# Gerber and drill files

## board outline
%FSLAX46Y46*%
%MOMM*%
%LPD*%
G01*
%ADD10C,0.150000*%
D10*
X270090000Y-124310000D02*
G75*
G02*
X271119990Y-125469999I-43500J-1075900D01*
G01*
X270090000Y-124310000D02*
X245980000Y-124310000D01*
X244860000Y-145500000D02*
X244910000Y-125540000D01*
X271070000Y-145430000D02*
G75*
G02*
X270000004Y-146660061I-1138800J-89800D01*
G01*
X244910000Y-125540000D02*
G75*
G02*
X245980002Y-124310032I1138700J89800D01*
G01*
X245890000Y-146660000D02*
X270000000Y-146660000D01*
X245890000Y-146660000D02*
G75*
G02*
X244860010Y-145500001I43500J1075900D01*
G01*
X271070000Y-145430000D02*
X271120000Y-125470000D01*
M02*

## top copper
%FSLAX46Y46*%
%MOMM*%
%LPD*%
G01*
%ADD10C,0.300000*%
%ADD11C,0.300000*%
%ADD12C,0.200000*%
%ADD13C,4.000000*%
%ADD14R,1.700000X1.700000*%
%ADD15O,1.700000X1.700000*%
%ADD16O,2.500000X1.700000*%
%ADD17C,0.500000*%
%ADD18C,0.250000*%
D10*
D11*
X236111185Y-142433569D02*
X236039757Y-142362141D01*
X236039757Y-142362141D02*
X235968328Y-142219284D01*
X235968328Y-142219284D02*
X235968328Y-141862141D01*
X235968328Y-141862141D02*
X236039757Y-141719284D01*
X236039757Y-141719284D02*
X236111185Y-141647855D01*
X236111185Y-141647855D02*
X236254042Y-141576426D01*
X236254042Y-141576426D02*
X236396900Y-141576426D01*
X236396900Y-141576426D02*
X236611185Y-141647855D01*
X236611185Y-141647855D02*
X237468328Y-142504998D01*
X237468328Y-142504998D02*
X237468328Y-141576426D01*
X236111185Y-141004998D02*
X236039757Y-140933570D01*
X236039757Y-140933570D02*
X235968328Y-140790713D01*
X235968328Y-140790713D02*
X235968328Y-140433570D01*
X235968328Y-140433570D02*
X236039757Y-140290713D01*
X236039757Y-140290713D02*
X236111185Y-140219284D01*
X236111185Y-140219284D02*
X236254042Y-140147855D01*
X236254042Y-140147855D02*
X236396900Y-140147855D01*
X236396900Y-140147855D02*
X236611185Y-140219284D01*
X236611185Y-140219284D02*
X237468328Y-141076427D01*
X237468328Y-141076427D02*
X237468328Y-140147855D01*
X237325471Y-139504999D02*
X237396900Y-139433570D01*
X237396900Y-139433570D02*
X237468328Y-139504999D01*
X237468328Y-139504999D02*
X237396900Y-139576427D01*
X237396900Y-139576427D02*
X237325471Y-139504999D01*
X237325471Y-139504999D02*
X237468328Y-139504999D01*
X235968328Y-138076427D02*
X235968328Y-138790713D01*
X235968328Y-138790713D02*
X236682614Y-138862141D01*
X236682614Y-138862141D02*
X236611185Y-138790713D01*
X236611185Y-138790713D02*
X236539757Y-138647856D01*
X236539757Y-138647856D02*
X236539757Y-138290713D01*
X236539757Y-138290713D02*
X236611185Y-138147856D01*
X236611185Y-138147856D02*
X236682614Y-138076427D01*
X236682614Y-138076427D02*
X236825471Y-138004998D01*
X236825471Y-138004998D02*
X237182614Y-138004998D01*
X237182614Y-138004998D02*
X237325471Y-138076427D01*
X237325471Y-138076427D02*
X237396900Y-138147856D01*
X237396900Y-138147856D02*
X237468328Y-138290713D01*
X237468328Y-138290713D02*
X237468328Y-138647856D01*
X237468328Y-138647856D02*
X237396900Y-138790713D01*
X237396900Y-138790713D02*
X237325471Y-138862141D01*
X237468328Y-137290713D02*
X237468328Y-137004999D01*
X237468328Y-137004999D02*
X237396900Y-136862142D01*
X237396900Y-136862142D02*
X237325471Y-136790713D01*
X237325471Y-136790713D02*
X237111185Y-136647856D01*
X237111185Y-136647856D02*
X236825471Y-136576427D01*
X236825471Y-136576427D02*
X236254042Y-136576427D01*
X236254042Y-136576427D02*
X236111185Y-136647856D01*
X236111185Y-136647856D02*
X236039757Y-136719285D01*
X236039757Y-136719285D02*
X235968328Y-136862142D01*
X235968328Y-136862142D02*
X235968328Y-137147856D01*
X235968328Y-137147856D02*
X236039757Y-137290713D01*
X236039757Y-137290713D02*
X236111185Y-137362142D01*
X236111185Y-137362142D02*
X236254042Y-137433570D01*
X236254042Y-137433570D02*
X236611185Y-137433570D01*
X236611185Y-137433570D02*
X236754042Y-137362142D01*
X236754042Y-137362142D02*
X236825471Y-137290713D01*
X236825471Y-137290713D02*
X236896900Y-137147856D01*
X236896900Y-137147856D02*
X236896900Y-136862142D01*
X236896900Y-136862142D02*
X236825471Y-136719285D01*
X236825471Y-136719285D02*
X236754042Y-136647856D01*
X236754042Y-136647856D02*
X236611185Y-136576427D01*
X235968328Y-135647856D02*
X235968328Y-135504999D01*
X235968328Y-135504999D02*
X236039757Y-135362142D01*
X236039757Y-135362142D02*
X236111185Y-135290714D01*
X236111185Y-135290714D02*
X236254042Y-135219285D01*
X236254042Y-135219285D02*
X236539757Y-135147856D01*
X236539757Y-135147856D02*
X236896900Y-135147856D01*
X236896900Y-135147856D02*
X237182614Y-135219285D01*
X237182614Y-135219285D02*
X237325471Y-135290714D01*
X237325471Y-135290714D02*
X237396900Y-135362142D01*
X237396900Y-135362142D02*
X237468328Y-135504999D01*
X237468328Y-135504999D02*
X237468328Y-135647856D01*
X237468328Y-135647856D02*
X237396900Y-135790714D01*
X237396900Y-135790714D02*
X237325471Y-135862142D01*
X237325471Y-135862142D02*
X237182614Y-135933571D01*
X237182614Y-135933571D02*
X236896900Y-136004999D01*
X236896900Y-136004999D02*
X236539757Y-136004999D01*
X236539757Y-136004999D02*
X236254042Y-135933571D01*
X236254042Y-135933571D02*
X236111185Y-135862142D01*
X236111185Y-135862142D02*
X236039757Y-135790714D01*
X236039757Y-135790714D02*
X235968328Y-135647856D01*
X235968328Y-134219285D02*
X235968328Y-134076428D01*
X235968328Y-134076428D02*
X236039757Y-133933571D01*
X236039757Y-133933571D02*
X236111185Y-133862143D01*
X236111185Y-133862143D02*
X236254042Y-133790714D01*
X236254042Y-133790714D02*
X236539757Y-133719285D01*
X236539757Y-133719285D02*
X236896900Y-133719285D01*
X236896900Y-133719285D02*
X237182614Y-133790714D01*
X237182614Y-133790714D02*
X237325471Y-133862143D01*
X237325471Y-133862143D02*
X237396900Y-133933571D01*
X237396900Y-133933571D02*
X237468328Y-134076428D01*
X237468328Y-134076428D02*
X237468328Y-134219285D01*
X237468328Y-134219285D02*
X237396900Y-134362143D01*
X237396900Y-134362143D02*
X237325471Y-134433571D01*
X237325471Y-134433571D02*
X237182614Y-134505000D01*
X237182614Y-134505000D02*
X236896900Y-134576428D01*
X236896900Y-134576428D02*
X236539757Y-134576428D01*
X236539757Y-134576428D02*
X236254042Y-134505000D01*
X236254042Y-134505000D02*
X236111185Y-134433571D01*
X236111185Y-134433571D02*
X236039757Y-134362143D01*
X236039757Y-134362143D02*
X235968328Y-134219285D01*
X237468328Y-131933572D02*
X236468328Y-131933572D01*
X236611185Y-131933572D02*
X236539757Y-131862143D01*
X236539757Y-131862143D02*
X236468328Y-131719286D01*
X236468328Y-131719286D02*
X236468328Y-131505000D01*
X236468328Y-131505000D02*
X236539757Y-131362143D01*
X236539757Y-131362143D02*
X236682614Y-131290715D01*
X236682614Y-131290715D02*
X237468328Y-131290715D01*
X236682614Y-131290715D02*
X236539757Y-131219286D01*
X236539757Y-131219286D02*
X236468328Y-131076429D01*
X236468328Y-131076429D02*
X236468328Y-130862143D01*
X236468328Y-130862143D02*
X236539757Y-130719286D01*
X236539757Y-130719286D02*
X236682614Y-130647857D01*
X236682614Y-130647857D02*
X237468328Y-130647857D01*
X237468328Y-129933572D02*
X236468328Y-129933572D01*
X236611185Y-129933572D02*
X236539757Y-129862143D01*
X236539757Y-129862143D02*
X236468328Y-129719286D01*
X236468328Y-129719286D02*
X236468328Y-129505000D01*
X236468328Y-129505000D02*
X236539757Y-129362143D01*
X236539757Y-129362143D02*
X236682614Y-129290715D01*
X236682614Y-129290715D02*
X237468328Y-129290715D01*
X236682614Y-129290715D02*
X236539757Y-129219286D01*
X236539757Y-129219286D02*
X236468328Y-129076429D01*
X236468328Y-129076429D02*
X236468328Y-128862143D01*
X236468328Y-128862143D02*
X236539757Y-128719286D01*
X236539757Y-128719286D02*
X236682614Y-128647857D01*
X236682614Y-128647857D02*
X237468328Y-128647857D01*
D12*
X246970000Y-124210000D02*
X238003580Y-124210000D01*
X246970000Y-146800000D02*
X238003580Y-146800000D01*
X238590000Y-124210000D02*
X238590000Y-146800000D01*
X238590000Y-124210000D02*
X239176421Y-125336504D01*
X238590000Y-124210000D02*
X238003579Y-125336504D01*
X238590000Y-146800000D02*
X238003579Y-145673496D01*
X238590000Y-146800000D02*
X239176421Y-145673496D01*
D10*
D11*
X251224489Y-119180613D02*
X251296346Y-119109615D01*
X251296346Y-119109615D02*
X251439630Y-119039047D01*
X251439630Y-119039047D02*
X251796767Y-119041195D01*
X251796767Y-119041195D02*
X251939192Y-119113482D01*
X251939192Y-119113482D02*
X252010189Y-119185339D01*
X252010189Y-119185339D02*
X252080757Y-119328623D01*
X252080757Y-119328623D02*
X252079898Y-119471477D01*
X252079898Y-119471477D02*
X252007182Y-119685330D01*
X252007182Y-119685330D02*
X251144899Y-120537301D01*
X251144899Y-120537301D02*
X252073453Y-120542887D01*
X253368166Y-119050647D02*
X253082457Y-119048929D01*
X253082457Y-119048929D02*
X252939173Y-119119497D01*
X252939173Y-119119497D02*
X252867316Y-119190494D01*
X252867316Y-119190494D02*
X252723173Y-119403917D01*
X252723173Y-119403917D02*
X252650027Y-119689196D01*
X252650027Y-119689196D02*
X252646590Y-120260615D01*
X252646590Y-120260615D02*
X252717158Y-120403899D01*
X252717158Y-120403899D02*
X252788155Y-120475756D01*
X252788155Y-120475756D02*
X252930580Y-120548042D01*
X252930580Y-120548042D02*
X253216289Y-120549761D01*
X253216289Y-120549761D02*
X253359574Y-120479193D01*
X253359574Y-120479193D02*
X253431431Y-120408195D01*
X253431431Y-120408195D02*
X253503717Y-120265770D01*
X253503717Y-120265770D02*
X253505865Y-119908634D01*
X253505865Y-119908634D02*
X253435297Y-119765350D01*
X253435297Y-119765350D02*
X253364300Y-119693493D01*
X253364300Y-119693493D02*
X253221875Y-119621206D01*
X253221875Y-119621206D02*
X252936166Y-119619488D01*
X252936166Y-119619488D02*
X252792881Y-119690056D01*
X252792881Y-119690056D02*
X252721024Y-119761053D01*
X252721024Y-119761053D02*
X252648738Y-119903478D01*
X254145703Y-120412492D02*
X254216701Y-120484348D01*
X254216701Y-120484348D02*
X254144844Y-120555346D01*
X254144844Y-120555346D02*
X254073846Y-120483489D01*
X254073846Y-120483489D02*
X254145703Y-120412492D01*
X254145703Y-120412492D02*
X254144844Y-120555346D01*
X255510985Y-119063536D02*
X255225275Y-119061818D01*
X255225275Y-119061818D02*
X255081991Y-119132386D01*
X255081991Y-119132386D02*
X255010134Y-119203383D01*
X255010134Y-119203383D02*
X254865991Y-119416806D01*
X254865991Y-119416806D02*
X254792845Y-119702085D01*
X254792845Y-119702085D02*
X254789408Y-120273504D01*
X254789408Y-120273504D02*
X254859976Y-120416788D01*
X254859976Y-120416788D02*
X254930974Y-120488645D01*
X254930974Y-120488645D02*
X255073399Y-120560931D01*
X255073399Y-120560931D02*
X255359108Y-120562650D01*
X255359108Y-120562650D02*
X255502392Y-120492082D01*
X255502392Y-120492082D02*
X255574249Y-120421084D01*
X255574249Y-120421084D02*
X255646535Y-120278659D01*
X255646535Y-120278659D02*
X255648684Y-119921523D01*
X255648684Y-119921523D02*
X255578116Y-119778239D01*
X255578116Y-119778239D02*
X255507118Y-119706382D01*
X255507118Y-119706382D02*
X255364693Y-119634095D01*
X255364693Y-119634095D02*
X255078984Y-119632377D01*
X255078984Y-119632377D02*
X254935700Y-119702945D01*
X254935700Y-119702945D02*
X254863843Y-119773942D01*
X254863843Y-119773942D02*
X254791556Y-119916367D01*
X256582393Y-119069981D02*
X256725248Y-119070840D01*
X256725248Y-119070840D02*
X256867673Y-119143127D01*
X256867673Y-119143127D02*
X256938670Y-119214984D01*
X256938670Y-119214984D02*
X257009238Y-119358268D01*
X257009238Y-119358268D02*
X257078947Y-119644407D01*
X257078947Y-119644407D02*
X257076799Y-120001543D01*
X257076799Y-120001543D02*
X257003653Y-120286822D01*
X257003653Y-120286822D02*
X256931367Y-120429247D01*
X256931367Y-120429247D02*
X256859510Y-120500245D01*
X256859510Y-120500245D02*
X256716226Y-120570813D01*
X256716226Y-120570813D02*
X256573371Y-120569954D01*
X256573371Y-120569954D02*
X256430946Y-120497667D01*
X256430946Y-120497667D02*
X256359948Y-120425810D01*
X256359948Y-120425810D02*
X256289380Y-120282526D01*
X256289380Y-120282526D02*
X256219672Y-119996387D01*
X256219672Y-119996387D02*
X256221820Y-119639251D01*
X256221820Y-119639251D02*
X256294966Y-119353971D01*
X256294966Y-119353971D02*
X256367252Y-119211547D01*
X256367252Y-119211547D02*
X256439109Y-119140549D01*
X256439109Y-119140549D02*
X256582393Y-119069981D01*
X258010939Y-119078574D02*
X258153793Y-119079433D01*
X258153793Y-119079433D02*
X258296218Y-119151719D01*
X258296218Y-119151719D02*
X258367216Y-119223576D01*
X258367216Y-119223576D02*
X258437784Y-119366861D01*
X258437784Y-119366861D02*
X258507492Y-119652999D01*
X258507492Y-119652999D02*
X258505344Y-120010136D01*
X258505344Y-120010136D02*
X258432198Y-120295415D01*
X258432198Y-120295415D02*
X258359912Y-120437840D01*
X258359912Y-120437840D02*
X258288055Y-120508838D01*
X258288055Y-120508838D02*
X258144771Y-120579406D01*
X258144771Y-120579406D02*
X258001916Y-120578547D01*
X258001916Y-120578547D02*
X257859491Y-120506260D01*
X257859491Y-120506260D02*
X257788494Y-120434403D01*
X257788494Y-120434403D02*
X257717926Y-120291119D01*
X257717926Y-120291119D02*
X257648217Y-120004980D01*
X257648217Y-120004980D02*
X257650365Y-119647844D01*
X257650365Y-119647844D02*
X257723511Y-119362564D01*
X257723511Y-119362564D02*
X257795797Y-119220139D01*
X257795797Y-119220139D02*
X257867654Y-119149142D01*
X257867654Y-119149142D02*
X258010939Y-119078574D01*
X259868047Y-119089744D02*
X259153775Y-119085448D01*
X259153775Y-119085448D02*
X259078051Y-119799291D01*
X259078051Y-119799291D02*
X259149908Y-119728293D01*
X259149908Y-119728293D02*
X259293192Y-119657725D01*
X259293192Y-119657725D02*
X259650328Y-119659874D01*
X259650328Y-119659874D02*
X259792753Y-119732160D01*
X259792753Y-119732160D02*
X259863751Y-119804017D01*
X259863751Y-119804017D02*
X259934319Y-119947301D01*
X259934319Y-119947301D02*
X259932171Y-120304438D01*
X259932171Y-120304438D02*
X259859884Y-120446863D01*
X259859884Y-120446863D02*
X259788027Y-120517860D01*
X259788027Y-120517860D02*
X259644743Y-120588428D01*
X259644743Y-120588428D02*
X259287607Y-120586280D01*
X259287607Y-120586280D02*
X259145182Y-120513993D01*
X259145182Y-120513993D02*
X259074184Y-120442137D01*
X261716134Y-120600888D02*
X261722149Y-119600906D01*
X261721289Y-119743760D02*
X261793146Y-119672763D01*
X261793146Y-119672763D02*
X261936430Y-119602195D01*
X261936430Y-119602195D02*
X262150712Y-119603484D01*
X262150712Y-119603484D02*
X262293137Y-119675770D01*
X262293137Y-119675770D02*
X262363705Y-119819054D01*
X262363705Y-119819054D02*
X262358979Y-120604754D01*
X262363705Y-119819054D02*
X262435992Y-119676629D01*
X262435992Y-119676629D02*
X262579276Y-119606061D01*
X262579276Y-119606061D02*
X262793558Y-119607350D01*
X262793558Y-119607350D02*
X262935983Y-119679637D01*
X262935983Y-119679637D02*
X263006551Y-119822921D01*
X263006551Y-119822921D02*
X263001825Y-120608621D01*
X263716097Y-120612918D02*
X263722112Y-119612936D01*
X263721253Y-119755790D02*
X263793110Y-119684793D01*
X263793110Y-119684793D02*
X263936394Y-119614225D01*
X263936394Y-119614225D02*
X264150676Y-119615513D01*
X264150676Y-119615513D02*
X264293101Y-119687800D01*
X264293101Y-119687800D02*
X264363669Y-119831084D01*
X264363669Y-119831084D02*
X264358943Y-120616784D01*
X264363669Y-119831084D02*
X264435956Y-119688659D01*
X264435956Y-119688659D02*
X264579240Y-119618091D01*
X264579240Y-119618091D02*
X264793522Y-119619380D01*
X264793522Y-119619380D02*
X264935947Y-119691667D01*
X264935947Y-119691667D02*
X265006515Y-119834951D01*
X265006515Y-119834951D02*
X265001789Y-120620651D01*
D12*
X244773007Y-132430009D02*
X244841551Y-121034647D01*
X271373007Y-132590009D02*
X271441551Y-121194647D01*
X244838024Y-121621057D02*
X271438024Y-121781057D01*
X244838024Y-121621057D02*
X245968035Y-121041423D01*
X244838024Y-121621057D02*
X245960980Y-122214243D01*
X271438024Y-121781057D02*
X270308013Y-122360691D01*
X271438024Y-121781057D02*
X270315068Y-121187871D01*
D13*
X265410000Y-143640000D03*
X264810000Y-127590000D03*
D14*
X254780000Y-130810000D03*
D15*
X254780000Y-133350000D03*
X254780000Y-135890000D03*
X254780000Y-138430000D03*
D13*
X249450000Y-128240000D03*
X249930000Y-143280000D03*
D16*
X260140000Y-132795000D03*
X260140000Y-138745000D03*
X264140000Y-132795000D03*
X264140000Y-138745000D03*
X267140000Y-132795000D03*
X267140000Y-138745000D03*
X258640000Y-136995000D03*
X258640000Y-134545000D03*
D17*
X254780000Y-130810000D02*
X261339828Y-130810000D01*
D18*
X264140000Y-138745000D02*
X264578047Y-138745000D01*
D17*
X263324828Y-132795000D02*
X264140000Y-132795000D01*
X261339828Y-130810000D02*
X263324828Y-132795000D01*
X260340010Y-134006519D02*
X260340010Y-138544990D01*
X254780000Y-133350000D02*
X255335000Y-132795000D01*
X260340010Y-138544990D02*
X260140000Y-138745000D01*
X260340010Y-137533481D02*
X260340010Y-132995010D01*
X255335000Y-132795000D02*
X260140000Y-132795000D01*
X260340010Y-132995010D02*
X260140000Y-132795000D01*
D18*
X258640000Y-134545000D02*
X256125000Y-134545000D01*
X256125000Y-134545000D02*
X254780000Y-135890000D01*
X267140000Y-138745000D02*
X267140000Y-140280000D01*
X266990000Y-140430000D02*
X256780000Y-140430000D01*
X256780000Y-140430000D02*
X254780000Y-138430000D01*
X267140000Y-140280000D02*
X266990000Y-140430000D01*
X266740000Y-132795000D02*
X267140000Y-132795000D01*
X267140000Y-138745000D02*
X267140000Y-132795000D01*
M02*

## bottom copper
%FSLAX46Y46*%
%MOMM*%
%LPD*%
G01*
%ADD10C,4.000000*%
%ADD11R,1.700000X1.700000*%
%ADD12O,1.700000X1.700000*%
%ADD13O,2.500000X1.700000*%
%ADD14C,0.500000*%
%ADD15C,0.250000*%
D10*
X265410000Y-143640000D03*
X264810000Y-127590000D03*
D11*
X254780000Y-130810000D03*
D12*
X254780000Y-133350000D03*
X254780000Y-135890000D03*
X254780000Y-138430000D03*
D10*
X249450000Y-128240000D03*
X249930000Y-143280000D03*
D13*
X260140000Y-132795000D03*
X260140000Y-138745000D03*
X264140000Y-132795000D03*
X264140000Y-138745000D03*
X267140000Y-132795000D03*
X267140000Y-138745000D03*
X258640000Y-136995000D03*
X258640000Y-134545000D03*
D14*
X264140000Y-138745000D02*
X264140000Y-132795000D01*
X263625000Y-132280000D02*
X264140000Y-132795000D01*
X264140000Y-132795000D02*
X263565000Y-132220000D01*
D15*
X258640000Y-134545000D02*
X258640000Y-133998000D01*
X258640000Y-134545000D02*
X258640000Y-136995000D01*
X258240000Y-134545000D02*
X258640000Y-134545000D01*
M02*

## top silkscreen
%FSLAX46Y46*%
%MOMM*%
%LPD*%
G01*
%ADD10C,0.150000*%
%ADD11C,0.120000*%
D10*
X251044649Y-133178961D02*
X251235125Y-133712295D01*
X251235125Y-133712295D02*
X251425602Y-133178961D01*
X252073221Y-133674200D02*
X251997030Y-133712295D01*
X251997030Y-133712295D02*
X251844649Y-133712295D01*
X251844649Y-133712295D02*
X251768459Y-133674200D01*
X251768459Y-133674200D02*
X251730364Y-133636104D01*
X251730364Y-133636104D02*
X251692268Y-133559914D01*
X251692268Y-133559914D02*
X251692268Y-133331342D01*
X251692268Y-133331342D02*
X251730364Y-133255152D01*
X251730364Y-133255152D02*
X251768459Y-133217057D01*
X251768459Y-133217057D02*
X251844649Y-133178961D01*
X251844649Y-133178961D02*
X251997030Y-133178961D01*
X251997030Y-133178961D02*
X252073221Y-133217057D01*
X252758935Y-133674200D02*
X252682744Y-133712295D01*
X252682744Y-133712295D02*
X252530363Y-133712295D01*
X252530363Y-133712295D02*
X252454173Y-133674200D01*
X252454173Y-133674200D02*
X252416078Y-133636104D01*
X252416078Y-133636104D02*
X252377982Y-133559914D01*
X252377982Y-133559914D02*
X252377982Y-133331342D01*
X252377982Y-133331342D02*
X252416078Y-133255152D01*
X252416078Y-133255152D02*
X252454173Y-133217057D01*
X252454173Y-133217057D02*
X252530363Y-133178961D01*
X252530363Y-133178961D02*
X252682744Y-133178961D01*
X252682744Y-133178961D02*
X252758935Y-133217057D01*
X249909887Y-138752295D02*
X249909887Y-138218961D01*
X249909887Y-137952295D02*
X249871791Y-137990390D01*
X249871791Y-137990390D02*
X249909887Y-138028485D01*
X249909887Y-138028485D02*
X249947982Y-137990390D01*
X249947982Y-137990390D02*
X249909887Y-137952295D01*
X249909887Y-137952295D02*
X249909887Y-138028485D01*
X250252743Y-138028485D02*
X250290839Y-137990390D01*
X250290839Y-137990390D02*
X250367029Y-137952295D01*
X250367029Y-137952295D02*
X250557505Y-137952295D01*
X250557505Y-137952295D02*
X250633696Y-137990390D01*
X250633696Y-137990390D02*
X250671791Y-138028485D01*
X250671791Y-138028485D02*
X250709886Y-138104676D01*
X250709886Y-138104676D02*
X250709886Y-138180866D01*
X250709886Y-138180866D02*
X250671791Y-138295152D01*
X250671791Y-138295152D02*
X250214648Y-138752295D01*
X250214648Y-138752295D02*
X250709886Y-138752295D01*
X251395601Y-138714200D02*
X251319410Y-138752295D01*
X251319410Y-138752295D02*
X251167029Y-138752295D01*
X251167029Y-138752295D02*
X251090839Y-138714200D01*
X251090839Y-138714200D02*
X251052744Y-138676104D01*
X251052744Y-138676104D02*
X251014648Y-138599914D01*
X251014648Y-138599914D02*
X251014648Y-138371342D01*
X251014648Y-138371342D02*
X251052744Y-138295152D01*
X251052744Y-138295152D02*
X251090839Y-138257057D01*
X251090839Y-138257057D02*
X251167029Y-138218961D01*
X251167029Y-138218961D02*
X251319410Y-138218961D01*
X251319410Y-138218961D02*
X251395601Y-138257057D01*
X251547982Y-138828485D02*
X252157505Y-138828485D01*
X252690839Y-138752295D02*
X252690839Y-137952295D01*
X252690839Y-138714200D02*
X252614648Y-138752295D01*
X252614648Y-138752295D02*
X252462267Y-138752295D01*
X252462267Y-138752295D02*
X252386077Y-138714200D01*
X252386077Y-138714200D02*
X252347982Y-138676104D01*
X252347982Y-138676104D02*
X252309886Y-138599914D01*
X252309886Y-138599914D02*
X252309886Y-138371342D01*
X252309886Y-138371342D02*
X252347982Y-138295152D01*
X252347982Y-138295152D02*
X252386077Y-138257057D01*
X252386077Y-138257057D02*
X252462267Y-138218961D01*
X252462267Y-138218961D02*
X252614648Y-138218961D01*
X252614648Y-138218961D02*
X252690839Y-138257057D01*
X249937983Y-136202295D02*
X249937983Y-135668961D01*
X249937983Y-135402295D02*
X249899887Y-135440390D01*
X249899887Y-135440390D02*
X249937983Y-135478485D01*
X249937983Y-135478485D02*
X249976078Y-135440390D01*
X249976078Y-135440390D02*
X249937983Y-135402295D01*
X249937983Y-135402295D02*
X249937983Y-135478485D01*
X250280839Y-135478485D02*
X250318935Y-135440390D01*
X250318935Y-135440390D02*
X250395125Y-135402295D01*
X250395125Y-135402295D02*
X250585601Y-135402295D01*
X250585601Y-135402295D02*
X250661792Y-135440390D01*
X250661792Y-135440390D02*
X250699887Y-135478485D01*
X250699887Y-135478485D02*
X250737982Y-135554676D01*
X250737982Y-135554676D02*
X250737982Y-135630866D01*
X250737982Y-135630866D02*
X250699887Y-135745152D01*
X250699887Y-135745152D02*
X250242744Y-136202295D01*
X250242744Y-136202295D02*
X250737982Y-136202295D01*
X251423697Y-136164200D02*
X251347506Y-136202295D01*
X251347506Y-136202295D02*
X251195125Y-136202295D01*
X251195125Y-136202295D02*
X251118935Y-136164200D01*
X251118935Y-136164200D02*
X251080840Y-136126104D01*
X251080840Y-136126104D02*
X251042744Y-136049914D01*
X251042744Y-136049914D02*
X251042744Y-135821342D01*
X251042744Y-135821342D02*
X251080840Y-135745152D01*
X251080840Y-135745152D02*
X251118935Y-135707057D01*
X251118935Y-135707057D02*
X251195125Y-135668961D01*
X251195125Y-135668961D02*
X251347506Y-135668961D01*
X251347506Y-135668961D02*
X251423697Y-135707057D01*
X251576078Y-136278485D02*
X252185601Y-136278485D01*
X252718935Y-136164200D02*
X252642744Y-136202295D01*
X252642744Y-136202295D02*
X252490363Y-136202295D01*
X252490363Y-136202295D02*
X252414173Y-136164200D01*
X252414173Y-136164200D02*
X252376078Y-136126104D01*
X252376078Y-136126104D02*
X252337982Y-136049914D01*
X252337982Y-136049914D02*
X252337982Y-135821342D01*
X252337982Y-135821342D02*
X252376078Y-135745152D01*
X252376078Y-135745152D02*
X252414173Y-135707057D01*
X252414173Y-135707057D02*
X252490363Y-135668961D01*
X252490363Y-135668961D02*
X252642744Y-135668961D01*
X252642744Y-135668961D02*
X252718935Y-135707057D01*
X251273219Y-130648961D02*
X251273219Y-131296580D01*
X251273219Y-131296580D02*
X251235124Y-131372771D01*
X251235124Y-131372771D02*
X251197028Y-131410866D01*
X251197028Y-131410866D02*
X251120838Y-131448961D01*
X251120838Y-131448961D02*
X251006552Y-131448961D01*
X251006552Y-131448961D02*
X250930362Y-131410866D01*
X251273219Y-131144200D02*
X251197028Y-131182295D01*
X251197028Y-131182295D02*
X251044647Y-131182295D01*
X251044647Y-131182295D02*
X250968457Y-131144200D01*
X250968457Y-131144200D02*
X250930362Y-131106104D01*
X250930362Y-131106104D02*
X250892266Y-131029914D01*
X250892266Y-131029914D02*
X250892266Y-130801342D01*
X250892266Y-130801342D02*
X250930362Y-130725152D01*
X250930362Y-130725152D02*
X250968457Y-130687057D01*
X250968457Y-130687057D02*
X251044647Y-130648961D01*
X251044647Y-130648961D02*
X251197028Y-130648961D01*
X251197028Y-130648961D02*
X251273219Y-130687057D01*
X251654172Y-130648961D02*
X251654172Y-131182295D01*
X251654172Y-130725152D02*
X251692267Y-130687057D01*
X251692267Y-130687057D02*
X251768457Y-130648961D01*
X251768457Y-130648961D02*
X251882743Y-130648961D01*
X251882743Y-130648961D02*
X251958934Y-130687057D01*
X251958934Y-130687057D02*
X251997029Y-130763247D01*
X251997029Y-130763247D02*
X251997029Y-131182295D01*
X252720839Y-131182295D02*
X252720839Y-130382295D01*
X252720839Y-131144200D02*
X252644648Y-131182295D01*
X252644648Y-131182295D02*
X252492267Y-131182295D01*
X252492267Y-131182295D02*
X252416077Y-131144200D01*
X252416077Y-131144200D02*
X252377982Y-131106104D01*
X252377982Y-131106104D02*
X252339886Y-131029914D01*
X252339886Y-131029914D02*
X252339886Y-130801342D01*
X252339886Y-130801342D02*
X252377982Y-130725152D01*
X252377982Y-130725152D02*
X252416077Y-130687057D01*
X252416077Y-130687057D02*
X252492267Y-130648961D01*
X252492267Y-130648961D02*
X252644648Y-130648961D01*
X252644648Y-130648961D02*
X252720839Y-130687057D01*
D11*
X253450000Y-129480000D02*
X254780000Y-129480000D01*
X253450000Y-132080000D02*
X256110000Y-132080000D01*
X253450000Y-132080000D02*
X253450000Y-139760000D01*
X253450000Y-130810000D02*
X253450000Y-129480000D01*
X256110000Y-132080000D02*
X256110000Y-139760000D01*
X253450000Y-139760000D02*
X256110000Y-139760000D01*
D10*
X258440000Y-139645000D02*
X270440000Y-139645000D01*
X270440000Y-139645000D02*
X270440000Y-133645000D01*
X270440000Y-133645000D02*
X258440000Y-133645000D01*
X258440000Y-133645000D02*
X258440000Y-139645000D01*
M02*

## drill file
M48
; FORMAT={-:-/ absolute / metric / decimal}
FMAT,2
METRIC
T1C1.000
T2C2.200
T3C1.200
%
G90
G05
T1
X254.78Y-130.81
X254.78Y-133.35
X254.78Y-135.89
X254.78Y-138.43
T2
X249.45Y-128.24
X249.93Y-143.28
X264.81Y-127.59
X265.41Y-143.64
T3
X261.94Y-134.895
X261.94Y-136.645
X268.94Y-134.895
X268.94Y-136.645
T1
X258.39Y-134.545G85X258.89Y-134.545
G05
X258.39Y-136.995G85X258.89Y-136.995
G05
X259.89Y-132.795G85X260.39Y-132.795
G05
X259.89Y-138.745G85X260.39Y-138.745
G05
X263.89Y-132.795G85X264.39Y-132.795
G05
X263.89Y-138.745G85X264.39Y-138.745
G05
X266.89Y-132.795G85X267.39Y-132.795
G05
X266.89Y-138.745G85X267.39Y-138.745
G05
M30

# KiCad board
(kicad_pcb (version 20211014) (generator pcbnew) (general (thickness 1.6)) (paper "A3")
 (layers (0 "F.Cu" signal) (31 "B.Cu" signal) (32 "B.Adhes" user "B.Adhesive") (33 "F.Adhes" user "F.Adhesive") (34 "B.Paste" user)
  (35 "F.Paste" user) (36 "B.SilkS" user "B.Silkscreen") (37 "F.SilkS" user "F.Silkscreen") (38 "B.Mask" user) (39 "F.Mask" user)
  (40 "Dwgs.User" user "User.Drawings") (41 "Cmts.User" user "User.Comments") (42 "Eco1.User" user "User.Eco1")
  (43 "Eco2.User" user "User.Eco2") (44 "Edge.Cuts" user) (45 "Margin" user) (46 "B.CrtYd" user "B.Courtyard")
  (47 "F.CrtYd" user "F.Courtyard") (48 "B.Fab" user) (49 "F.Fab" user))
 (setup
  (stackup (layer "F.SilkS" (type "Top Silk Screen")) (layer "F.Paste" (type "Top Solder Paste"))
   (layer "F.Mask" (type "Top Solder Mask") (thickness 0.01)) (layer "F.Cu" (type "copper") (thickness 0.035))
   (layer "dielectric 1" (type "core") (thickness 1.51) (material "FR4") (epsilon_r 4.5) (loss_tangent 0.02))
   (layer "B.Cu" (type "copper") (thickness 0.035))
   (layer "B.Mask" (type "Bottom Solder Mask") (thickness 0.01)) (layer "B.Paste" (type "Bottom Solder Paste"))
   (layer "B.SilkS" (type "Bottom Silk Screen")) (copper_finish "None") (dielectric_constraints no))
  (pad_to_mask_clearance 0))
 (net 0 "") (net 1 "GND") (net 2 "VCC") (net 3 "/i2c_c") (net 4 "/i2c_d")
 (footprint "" (layer "F.Cu") (at 265.41 143.64)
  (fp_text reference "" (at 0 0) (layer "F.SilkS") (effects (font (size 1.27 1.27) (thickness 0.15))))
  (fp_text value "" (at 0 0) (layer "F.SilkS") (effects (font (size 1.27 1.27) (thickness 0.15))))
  (pad "" thru_hole circle locked (at 0 0 180) (size 4 4) (drill 2.2) (layers F&B.Cu *.Mask "Dwgs.User")))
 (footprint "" (layer "F.Cu") (at 264.81 127.59)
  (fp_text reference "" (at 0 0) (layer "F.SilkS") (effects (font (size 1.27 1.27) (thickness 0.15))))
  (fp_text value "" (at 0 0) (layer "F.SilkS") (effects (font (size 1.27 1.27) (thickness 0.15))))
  (pad "" thru_hole circle locked (at 0 0 180) (size 4 4) (drill 2.2) (layers F&B.Cu *.Mask "Dwgs.User")))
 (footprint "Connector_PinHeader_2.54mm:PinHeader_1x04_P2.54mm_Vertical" (layer "F.Cu") (at 254.78 130.81)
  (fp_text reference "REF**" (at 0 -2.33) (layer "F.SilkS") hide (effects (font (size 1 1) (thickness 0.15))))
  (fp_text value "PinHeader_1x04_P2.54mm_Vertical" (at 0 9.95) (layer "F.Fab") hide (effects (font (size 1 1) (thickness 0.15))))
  (fp_line (start -1.33 -1.33) (end 0 -1.33) (layer "F.SilkS") (width 0.12))
  (fp_line (start -1.33 1.27) (end 1.33 1.27) (layer "F.SilkS") (width 0.12))
  (fp_line (start -1.33 1.27) (end -1.33 8.95) (layer "F.SilkS") (width 0.12))
  (fp_line (start -1.33 0) (end -1.33 -1.33) (layer "F.SilkS") (width 0.12))
  (fp_line (start 1.33 1.27) (end 1.33 8.95) (layer "F.SilkS") (width 0.12))
  (fp_line (start -1.33 8.95) (end 1.33 8.95) (layer "F.SilkS") (width 0.12))
  (pad "1" thru_hole rect (at 0 0) (size 1.7 1.7) (drill 1) (layers *.Cu *.Mask) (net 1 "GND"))
  (pad "2" thru_hole oval (at 0 2.54) (size 1.7 1.7) (drill 1) (layers *.Cu *.Mask) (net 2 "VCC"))
  (pad "3" thru_hole oval (at 0 5.08) (size 1.7 1.7) (drill 1) (layers *.Cu *.Mask) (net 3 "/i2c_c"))
  (pad "4" thru_hole oval (at 0 7.62) (size 1.7 1.7) (drill 1) (layers *.Cu *.Mask) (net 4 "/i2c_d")))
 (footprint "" (layer "F.Cu") (at 249.45 128.24)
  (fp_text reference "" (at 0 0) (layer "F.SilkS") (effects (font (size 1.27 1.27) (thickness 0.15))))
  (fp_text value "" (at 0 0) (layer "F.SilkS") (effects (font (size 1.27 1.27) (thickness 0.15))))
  (pad "" thru_hole circle locked (at 0 0 180) (size 4 4) (drill 2.2) (layers F&B.Cu *.Mask "Dwgs.User")))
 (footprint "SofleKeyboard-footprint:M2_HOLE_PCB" (layer "B.Cu") (at 249.93 143.28 180)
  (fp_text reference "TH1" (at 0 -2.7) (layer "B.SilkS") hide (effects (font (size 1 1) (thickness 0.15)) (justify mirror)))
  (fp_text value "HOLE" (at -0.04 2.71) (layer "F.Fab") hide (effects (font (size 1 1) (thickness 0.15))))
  (pad "" thru_hole circle locked (at 0 0 180) (size 4 4) (drill 2.2) (layers F&B.Cu *.Mask "Dwgs.User")))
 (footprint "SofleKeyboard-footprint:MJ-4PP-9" (layer "B.Cu") (at 270.44 134.895 90)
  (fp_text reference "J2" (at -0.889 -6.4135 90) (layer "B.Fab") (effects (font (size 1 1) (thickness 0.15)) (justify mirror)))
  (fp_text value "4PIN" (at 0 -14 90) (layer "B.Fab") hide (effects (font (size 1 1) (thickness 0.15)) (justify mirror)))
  (fp_line (start -4.75 -12) (end -4.75 0) (layer "F.SilkS") (width 0.15))
  (fp_line (start -4.75 0) (end 1.25 0) (layer "F.SilkS") (width 0.15))
  (fp_line (start 1.25 0) (end 1.25 -12) (layer "F.SilkS") (width 0.15))
  (fp_line (start 1.25 -12) (end -4.75 -12) (layer "F.SilkS") (width 0.15))
  (pad "" np_thru_hole circle locked (at 0 -1.5 90) (size 1.2 1.2) (drill 1.2) (layers F&B.Cu *.Mask "B.SilkS"))
  (pad "" np_thru_hole circle locked (at -1.75 -1.5 90) (size 1.2 1.2) (drill 1.2) (layers F&B.Cu *.Mask "B.SilkS"))
  (pad "" np_thru_hole circle locked (at -1.75 -8.5 90) (size 1.2 1.2) (drill 1.2) (layers F&B.Cu *.Mask "B.SilkS"))
  (pad "" np_thru_hole circle locked (at 0 -8.5 90) (size 1.2 1.2) (drill 1.2) (layers F&B.Cu *.Mask "B.SilkS"))
  (pad "1" thru_hole oval locked (at 2.1 -10.3 90) (size 1.7 2.5) (drill oval 1 1.5) (layers F&B.Cu *.Mask "B.SilkS") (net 2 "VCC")
   (clearance 0.15))
  (pad "1" thru_hole oval locked (at -3.85 -10.3 90) (size 1.7 2.5) (drill oval 1 1.5) (layers F&B.Cu *.Mask "B.SilkS") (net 2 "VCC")
   (clearance 0.15))
  (pad "2" thru_hole oval locked (at 2.1 -6.3 90) (size 1.7 2.5) (drill oval 1 1.5) (layers F&B.Cu *.Mask "B.SilkS") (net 1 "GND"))
  (pad "2" thru_hole oval locked (at -3.85 -6.3 90) (size 1.7 2.5) (drill oval 1 1.5) (layers F&B.Cu *.Mask "B.SilkS") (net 1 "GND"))
  (pad "3" thru_hole oval locked (at 2.1 -3.3 90) (size 1.7 2.5) (drill oval 1 1.5) (layers *.Cu *.Mask "B.SilkS") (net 4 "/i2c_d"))
  (pad "3" thru_hole oval locked (at -3.85 -3.3 90) (size 1.7 2.5) (drill oval 1 1.5) (layers *.Cu *.Mask "B.SilkS") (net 4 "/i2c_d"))
  (pad "4" thru_hole oval locked (at -2.1 -11.8 90) (size 1.7 2.5) (drill oval 1 1.5) (layers *.Cu *.Mask "B.SilkS") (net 3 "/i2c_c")
   (clearance 0.15))
  (pad "4" thru_hole oval locked (at 0.35 -11.8 90) (size 1.7 2.5) (drill oval 1 1.5) (layers *.Cu *.Mask "B.SilkS") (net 3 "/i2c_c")
   (clearance 0.15)))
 (gr_arc (start 270.09 124.31) (mid 270.851681 124.670962) (end 271.12 125.47) (layer "Edge.Cuts") (width 0.15))
 (gr_line (start 270.09 124.31) (end 245.98 124.31) (layer "Edge.Cuts") (width 0.15))
 (gr_line (start 244.86 145.5) (end 244.91 125.54) (layer "Edge.Cuts") (width 0.15))
 (gr_arc (start 271.07 145.43) (mid 270.793076 146.269496) (end 270 146.66) (layer "Edge.Cuts") (width 0.15))
 (gr_arc (start 244.91 125.54) (mid 245.186912 124.700487) (end 245.98 124.31) (layer "Edge.Cuts") (width 0.15))
 (gr_line (start 245.89 146.66) (end 270 146.66) (layer "Edge.Cuts") (width 0.15))
 (gr_arc (start 245.89 146.66) (mid 245.128308 146.299045) (end 244.86 145.5) (layer "Edge.Cuts") (width 0.15))
 (gr_line (start 271.07 145.43) (end 271.12 125.47) (layer "Edge.Cuts") (width 0.15))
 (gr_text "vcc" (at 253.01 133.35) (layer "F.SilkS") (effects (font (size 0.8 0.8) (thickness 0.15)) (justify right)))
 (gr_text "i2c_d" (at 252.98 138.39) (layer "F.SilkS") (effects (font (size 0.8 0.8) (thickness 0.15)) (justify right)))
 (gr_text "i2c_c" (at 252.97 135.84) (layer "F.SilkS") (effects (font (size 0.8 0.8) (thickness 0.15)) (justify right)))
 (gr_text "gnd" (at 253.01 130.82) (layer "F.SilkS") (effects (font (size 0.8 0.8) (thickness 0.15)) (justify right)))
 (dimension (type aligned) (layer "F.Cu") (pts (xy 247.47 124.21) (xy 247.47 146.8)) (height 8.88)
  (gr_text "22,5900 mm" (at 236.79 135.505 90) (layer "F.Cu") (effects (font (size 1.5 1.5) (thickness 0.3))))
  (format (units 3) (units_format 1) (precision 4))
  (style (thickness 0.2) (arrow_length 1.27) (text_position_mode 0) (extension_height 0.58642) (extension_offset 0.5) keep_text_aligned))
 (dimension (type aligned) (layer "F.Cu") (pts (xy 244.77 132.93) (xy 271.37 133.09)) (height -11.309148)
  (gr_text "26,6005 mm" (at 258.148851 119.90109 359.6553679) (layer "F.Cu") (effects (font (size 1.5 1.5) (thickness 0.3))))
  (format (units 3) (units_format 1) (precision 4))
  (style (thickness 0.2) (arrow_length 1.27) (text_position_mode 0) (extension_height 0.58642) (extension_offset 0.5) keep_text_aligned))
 (segment (start 254.78 130.81) (end 261.339828 130.81) (width 0.5) (layer "F.Cu") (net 1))
 (segment (start 264.14 138.745) (end 264.578047 138.745) (width 0.25) (layer "F.Cu") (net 1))
 (segment (start 263.324828 132.795) (end 264.14 132.795) (width 0.5) (layer "F.Cu") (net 1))
 (segment (start 261.339828 130.81) (end 263.324828 132.795) (width 0.5) (layer "F.Cu") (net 1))
 (segment (start 264.14 138.745) (end 264.14 132.795) (width 0.5) (layer "B.Cu") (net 1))
 (segment (start 263.625 132.28) (end 264.14 132.795) (width 0.5) (layer "B.Cu") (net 1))
 (segment (start 264.14 132.795) (end 263.565 132.22) (width 0.5) (layer "B.Cu") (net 1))
 (segment (start 260.34001 134.006519) (end 260.34001 138.54499) (width 0.5) (layer "F.Cu") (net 2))
 (segment (start 254.78 133.35) (end 255.335 132.795) (width 0.5) (layer "F.Cu") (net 2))
 (segment (start 260.34001 138.54499) (end 260.14 138.745) (width 0.5) (layer "F.Cu") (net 2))
 (segment (start 260.34001 137.533481) (end 260.34001 132.99501) (width 0.5) (layer "F.Cu") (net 2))
 (segment (start 255.335 132.795) (end 260.14 132.795) (width 0.5) (layer "F.Cu") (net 2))
 (segment (start 260.34001 132.99501) (end 260.14 132.795) (width 0.5) (layer "F.Cu") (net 2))
 (segment (start 258.64 134.545) (end 256.125 134.545) (width 0.25) (layer "F.Cu") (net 3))
 (segment (start 256.125 134.545) (end 254.78 135.89) (width 0.25) (layer "F.Cu") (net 3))
 (segment (start 258.64 134.545) (end 258.64 133.998) (width 0.25) (layer "B.Cu") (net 3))
 (segment (start 258.64 134.545) (end 258.64 136.995) (width 0.25) (layer "B.Cu") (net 3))
 (segment (start 258.24 134.545) (end 258.64 134.545) (width 0.25) (layer "B.Cu") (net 3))
 (segment (start 267.14 138.745) (end 267.14 140.28) (width 0.25) (layer "F.Cu") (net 4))
 (segment (start 266.99 140.43) (end 256.78 140.43) (width 0.25) (layer "F.Cu") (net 4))
 (segment (start 256.78 140.43) (end 254.78 138.43) (width 0.25) (layer "F.Cu") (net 4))
 (segment (start 267.14 140.28) (end 266.99 140.43) (width 0.25) (layer "F.Cu") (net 4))
 (segment (start 266.74 132.795) (end 267.14 132.795) (width 0.25) (layer "F.Cu") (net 4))
 (segment (start 267.14 138.745) (end 267.14 132.795) (width 0.25) (layer "F.Cu") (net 4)))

